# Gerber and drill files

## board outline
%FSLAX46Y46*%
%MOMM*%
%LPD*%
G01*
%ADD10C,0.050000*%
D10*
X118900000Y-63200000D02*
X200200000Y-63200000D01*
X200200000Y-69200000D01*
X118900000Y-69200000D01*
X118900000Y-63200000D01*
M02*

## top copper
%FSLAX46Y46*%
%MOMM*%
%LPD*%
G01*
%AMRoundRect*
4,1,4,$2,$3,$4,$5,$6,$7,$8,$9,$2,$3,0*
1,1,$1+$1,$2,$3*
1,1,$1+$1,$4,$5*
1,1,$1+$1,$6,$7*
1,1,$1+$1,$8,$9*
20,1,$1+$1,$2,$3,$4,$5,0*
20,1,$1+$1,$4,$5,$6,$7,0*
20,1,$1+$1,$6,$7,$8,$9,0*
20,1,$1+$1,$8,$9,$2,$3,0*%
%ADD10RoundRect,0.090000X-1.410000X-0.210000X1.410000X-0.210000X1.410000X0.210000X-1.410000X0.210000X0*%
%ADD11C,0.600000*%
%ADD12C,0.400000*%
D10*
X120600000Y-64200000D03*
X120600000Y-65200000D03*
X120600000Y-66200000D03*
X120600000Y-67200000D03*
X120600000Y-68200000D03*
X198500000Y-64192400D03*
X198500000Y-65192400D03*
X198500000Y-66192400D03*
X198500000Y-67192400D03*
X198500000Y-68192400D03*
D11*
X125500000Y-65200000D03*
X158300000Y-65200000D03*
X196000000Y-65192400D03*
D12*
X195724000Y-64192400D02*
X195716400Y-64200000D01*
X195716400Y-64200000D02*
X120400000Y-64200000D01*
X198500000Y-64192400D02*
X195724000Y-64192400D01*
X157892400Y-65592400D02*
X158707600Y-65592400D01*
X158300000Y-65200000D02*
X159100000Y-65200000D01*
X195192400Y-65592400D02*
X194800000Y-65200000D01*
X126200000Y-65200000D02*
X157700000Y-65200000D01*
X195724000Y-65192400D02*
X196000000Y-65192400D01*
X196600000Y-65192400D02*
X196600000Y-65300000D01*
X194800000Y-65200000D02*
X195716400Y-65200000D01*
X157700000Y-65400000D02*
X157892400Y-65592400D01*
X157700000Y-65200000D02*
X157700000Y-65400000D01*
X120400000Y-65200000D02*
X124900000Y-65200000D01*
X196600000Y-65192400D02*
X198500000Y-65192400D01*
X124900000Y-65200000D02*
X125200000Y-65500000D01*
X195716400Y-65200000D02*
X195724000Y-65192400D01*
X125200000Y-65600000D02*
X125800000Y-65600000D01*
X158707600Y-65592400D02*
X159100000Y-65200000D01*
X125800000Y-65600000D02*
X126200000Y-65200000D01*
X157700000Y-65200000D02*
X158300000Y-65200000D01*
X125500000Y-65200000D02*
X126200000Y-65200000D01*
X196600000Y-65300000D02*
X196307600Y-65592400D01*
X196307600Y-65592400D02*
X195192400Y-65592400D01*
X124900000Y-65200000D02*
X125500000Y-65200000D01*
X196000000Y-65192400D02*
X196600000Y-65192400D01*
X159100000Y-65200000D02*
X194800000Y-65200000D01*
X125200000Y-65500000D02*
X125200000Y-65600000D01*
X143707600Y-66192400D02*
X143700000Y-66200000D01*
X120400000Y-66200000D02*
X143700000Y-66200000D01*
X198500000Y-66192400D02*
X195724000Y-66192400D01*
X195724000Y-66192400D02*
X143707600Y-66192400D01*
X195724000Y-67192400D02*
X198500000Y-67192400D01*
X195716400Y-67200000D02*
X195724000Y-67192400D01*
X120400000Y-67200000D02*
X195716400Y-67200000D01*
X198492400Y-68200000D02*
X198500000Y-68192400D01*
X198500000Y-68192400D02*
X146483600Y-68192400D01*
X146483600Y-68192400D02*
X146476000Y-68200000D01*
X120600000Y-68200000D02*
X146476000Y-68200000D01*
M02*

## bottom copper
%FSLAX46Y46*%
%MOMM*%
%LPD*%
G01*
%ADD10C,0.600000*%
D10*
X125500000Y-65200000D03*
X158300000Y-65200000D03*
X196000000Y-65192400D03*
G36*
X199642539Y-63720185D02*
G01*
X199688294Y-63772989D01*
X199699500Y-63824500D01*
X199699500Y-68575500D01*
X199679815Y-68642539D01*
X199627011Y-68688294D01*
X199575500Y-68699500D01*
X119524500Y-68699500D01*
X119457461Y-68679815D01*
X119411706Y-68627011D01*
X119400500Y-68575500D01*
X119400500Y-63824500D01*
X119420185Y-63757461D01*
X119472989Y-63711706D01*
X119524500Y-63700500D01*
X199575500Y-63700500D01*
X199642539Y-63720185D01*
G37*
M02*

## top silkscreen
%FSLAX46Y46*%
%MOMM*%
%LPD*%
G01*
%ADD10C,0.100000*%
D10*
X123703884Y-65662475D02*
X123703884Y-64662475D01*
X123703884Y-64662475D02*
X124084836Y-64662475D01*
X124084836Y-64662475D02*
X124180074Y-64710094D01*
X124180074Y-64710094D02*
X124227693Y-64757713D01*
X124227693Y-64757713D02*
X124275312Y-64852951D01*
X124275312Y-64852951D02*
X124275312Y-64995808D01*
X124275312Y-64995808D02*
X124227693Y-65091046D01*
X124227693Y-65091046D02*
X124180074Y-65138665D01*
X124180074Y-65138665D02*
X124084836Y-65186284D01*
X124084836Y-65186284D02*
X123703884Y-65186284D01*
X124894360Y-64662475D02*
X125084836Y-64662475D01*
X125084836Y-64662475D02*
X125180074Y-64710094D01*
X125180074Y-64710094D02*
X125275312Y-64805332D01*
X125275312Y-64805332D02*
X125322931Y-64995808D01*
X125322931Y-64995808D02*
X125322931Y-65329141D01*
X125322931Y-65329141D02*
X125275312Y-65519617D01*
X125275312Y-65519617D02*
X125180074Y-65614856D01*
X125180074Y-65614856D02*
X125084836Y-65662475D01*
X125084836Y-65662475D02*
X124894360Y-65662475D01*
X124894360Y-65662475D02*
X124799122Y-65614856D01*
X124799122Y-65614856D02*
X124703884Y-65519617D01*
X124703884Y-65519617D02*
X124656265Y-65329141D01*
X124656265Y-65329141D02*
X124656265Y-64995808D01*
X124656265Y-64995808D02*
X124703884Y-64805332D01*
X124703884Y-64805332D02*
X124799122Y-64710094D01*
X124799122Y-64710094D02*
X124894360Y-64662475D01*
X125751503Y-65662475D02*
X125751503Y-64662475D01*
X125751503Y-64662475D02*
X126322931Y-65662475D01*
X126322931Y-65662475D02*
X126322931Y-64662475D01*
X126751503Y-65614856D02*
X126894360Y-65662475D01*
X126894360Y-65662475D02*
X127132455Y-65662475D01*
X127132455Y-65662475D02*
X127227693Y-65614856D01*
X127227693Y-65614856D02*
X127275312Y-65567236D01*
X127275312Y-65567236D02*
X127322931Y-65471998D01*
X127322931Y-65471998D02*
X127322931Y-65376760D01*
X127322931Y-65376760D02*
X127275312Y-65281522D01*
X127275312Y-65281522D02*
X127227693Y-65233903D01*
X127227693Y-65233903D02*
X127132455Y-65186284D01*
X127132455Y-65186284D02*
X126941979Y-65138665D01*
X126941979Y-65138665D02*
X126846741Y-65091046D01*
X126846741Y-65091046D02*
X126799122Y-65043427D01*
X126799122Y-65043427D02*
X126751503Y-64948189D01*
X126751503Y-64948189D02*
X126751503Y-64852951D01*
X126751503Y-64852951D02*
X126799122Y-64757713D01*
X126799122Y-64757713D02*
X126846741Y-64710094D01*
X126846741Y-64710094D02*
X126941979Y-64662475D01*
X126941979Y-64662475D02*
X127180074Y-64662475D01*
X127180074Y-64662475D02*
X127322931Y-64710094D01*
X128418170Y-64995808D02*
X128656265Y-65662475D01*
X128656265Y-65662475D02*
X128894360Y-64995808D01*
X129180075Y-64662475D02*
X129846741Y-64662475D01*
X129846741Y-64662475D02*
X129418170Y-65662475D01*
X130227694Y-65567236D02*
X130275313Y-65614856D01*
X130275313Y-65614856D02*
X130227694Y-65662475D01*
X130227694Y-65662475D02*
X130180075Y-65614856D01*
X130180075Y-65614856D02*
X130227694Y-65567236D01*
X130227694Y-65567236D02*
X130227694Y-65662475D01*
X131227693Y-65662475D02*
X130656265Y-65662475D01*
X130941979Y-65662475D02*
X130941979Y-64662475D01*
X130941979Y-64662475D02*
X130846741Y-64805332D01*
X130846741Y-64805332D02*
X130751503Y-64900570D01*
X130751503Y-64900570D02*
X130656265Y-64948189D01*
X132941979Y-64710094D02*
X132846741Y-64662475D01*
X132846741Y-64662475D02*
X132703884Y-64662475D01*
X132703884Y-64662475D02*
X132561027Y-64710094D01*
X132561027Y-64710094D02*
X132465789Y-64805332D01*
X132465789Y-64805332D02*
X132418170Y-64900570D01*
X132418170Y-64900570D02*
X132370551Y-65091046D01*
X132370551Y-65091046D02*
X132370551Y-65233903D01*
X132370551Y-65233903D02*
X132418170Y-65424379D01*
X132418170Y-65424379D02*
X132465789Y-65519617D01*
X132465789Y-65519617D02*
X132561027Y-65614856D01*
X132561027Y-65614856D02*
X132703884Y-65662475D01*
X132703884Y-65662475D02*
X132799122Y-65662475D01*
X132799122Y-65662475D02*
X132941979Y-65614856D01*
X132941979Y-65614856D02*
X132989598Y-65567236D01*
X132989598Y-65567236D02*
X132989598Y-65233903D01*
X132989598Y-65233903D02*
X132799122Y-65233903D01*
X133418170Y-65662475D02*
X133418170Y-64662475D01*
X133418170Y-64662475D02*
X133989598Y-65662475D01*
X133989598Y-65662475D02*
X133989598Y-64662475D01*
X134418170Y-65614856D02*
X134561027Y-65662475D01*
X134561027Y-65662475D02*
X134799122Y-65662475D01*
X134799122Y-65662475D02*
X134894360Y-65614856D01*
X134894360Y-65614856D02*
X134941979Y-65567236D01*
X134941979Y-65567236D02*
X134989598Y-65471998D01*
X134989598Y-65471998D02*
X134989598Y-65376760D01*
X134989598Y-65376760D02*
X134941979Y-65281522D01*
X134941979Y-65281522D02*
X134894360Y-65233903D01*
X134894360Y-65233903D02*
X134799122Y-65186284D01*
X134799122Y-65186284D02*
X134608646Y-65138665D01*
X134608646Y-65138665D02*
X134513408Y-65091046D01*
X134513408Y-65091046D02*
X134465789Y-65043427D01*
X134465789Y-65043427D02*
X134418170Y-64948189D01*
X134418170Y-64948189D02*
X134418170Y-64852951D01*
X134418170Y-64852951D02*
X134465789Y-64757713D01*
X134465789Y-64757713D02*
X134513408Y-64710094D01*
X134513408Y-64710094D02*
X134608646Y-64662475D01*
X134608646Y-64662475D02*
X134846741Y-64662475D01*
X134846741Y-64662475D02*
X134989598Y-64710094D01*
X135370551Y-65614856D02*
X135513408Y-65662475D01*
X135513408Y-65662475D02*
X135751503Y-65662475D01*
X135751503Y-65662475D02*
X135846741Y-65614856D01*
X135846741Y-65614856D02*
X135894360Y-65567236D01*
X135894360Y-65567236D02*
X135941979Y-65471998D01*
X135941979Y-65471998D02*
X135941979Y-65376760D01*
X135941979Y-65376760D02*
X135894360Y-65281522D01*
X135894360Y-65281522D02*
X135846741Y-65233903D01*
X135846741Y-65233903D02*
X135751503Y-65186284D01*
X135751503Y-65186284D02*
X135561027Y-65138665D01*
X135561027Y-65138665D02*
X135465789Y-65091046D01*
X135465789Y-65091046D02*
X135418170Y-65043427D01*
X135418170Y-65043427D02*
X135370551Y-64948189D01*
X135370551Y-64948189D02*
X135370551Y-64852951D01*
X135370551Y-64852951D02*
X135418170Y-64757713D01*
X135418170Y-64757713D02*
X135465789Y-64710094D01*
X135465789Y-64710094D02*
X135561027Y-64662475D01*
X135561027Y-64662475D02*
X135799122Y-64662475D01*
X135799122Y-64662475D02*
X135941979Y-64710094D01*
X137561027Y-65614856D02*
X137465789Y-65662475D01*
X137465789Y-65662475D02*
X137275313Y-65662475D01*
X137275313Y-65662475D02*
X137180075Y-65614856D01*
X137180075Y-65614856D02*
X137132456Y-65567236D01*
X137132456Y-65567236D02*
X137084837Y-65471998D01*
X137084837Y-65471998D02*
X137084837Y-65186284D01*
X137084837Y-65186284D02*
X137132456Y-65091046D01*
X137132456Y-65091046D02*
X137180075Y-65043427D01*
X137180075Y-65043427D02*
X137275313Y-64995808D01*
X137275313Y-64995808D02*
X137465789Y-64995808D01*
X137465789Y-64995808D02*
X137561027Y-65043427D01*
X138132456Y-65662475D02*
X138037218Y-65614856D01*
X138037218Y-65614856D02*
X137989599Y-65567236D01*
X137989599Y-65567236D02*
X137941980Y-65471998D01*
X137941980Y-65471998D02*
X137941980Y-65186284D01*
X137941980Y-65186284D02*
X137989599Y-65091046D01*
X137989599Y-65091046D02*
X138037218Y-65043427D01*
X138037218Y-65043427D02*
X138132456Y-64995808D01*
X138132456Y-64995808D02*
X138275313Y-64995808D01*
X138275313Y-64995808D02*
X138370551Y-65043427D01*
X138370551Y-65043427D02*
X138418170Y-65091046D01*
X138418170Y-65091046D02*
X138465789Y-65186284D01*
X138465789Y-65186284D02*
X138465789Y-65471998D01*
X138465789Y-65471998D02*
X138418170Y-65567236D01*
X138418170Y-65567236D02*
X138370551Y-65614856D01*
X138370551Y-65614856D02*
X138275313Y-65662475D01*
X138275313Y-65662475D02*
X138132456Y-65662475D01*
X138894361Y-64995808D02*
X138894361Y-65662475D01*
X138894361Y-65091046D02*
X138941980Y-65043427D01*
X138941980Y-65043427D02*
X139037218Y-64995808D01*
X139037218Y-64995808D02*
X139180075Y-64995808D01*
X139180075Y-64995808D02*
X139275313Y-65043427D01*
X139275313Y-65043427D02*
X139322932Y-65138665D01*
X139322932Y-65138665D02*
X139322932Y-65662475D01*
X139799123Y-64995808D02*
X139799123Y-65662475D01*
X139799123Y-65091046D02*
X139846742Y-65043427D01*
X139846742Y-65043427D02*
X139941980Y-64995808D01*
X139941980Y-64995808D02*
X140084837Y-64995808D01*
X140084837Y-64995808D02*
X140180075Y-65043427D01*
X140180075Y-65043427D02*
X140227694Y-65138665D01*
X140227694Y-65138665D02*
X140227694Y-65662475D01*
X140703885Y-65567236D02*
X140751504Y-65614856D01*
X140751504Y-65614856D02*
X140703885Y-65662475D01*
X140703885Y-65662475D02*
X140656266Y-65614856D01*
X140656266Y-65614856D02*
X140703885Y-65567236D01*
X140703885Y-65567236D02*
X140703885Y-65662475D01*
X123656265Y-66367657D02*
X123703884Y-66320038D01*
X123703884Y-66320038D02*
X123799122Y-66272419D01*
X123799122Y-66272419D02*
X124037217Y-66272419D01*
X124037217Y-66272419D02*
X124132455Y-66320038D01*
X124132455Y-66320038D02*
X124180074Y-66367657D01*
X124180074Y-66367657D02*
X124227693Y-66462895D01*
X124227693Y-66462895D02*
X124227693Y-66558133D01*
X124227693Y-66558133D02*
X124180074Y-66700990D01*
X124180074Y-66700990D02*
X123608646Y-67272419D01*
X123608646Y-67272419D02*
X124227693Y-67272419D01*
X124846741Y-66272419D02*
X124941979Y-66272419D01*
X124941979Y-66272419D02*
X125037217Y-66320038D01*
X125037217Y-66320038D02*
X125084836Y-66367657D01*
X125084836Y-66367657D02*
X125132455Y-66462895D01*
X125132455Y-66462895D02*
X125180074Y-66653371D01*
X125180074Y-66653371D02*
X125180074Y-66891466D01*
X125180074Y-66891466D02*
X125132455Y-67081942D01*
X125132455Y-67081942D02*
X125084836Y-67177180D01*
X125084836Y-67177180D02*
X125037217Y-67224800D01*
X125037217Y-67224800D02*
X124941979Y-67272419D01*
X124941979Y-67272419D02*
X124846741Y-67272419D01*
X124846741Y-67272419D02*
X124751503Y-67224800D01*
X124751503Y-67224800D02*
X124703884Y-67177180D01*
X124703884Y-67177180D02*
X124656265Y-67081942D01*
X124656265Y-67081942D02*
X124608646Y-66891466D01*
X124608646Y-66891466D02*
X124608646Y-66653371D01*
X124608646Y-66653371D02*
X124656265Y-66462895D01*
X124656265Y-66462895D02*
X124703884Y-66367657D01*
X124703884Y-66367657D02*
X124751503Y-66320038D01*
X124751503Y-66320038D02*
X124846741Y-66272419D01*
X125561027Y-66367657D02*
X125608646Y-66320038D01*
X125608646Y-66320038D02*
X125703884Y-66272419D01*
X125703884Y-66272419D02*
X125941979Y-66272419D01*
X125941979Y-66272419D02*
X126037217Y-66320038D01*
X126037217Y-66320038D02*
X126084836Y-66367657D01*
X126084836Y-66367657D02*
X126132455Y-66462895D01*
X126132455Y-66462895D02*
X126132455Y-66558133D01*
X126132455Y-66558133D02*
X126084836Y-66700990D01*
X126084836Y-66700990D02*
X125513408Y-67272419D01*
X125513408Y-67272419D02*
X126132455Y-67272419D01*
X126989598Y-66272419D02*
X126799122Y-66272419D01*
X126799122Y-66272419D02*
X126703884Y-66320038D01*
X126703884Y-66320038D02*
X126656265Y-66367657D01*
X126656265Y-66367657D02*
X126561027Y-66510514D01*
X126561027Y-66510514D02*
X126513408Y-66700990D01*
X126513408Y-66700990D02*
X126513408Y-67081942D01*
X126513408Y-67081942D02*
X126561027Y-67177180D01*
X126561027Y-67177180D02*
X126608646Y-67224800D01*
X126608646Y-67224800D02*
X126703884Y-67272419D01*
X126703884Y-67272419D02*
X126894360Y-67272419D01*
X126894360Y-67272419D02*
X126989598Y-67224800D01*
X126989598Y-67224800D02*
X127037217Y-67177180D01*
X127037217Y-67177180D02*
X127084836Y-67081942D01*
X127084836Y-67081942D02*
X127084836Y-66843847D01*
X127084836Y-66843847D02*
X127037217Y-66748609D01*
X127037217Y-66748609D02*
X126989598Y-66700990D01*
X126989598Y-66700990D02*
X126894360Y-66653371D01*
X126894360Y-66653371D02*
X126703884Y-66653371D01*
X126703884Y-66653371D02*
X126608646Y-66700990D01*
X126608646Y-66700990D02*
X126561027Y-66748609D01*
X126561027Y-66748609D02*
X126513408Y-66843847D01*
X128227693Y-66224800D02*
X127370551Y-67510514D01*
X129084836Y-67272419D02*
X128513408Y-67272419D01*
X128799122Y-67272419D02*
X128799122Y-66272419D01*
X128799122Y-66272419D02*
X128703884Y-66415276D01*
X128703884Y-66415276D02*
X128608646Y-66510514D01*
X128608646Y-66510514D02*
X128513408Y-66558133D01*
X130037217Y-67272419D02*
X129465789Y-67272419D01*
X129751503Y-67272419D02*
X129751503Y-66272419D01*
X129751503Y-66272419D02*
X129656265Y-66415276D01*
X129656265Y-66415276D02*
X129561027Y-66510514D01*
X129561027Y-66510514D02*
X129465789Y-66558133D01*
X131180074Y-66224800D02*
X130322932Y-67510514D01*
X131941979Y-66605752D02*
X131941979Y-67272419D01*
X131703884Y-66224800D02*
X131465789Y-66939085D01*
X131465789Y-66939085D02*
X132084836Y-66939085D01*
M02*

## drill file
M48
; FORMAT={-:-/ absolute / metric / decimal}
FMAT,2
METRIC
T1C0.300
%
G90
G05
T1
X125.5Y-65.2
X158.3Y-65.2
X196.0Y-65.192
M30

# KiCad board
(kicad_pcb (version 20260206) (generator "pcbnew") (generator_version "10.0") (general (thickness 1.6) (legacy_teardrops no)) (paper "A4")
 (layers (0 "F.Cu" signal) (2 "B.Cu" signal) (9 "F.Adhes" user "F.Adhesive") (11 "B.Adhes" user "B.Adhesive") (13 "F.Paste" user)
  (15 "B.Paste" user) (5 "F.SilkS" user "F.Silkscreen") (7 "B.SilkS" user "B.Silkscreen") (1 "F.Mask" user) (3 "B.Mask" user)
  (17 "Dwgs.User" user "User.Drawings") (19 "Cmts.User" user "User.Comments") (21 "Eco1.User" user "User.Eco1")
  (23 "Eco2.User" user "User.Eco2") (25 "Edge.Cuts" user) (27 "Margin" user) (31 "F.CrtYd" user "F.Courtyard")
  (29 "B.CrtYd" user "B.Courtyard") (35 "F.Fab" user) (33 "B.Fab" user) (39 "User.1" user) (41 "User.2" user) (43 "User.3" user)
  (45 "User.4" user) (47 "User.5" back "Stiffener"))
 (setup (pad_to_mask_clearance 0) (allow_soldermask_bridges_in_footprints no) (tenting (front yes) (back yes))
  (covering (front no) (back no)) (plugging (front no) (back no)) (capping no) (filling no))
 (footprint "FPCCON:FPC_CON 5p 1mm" (layer "F.Cu") (at 120.6 66.2)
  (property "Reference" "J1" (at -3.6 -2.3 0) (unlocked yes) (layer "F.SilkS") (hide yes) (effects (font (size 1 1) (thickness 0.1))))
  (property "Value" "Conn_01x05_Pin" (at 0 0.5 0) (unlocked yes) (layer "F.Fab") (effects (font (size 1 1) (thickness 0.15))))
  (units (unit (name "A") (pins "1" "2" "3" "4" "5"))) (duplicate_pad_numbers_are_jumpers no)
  (pad "1" smd roundrect (at 0 -2) (size 3 0.6) (layers "F.Cu" "F.Mask" "F.Paste") (roundrect_rratio 0.15) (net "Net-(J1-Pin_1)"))
  (pad "2" smd roundrect (at 0 -1) (size 3 0.6) (layers "F.Cu" "F.Mask" "F.Paste") (roundrect_rratio 0.15) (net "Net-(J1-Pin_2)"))
  (pad "3" smd roundrect (at 0 0) (size 3 0.6) (layers "F.Cu" "F.Mask" "F.Paste") (roundrect_rratio 0.15) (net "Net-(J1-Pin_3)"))
  (pad "4" smd roundrect (at 0 1) (size 3 0.6) (layers "F.Cu" "F.Mask" "F.Paste") (roundrect_rratio 0.15) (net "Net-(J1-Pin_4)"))
  (pad "5" smd roundrect (at 0 2) (size 3 0.6) (layers "F.Cu" "F.Mask" "F.Paste") (roundrect_rratio 0.15) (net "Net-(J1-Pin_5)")))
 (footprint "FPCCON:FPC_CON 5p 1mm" (layer "F.Cu") (at 198.5 66.1924)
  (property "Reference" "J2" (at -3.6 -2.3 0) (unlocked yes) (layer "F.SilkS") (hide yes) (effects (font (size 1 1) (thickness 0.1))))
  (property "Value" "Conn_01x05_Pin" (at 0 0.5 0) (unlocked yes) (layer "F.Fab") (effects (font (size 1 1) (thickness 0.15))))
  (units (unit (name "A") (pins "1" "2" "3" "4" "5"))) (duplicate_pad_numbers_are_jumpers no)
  (pad "1" smd roundrect (at 0 -2) (size 3 0.6) (layers "F.Cu" "F.Mask" "F.Paste") (roundrect_rratio 0.15) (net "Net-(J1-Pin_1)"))
  (pad "2" smd roundrect (at 0 -1) (size 3 0.6) (layers "F.Cu" "F.Mask" "F.Paste") (roundrect_rratio 0.15) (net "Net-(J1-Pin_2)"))
  (pad "3" smd roundrect (at 0 0) (size 3 0.6) (layers "F.Cu" "F.Mask" "F.Paste") (roundrect_rratio 0.15) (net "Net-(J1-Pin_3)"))
  (pad "4" smd roundrect (at 0 1) (size 3 0.6) (layers "F.Cu" "F.Mask" "F.Paste") (roundrect_rratio 0.15) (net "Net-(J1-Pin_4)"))
  (pad "5" smd roundrect (at 0 2) (size 3 0.6) (layers "F.Cu" "F.Mask" "F.Paste") (roundrect_rratio 0.15) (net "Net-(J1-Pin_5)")))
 (gr_rect (start 118.9 63.2) (end 200.2 69.2) (stroke (width 0.05) (type default)) (fill no) (layer "Edge.Cuts"))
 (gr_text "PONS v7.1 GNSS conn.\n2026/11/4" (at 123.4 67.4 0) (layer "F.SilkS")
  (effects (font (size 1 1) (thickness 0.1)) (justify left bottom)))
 (segment (start 195.724 64.1924) (end 195.7164 64.2) (width 0.4) (layer "F.Cu") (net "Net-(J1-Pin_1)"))
 (segment (start 195.7164 64.2) (end 120.4 64.2) (width 0.4) (layer "F.Cu") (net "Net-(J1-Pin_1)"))
 (segment (start 198.5 64.1924) (end 195.724 64.1924) (width 0.4) (layer "F.Cu") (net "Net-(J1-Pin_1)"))
 (segment (start 157.8924 65.5924) (end 158.7076 65.5924) (width 0.4) (layer "F.Cu") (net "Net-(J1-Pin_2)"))
 (segment (start 158.3 65.2) (end 159.1 65.2) (width 0.4) (layer "F.Cu") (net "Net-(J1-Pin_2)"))
 (segment (start 195.1924 65.5924) (end 194.8 65.2) (width 0.4) (layer "F.Cu") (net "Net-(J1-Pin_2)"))
 (segment (start 126.2 65.2) (end 157.7 65.2) (width 0.4) (layer "F.Cu") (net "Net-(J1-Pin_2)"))
 (segment (start 195.724 65.1924) (end 196 65.1924) (width 0.4) (layer "F.Cu") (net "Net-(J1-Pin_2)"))
 (segment (start 196.6 65.1924) (end 196.6 65.3) (width 0.4) (layer "F.Cu") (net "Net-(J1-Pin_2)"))
 (segment (start 194.8 65.2) (end 195.7164 65.2) (width 0.4) (layer "F.Cu") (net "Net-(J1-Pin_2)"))
 (segment (start 157.7 65.4) (end 157.8924 65.5924) (width 0.4) (layer "F.Cu") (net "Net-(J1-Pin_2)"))
 (segment (start 157.7 65.2) (end 157.7 65.4) (width 0.4) (layer "F.Cu") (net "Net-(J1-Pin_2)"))
 (segment (start 120.4 65.2) (end 124.9 65.2) (width 0.4) (layer "F.Cu") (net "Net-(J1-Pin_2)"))
 (segment (start 196.6 65.1924) (end 198.5 65.1924) (width 0.4) (layer "F.Cu") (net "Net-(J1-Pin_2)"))
 (segment (start 124.9 65.2) (end 125.2 65.5) (width 0.4) (layer "F.Cu") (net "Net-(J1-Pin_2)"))
 (segment (start 195.7164 65.2) (end 195.724 65.1924) (width 0.4) (layer "F.Cu") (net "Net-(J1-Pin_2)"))
 (segment (start 125.2 65.6) (end 125.8 65.6) (width 0.4) (layer "F.Cu") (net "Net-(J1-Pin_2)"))
 (segment (start 158.7076 65.5924) (end 159.1 65.2) (width 0.4) (layer "F.Cu") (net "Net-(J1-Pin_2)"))
 (segment (start 125.8 65.6) (end 126.2 65.2) (width 0.4) (layer "F.Cu") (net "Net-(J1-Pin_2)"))
 (segment (start 157.7 65.2) (end 158.3 65.2) (width 0.4) (layer "F.Cu") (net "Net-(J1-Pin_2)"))
 (segment (start 125.5 65.2) (end 126.2 65.2) (width 0.4) (layer "F.Cu") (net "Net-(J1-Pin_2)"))
 (segment (start 196.6 65.3) (end 196.3076 65.5924) (width 0.4) (layer "F.Cu") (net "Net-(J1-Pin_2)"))
 (segment (start 196.3076 65.5924) (end 195.1924 65.5924) (width 0.4) (layer "F.Cu") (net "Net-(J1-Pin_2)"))
 (segment (start 124.9 65.2) (end 125.5 65.2) (width 0.4) (layer "F.Cu") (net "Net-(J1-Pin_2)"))
 (segment (start 196 65.1924) (end 196.6 65.1924) (width 0.4) (layer "F.Cu") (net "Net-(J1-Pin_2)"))
 (segment (start 159.1 65.2) (end 194.8 65.2) (width 0.4) (layer "F.Cu") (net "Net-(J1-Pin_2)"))
 (segment (start 125.2 65.5) (end 125.2 65.6) (width 0.4) (layer "F.Cu") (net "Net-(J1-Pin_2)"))
 (via (at 125.5 65.2) (size 0.6) (drill 0.3) (layers "F.Cu" "B.Cu") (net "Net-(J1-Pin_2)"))
 (via (at 158.3 65.2) (size 0.6) (drill 0.3) (layers "F.Cu" "B.Cu") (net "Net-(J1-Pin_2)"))
 (via (at 196 65.1924) (size 0.6) (drill 0.3) (layers "F.Cu" "B.Cu") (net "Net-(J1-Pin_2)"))
 (segment (start 143.7076 66.1924) (end 143.7 66.2) (width 0.4) (layer "F.Cu") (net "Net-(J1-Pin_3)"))
 (segment (start 120.4 66.2) (end 143.7 66.2) (width 0.4) (layer "F.Cu") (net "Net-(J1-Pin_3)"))
 (segment (start 198.5 66.1924) (end 195.724 66.1924) (width 0.4) (layer "F.Cu") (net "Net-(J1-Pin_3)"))
 (segment (start 195.724 66.1924) (end 143.7076 66.1924) (width 0.4) (layer "F.Cu") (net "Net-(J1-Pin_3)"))
 (segment (start 195.724 67.1924) (end 198.5 67.1924) (width 0.4) (layer "F.Cu") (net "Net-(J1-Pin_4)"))
 (segment (start 195.7164 67.2) (end 195.724 67.1924) (width 0.4) (layer "F.Cu") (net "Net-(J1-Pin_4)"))
 (segment (start 120.4 67.2) (end 195.7164 67.2) (width 0.4) (layer "F.Cu") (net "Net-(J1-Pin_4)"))
 (segment (start 198.4924 68.2) (end 198.5 68.1924) (width 0.4) (layer "F.Cu") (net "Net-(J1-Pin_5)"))
 (segment (start 198.5 68.1924) (end 146.4836 68.1924) (width 0.4) (layer "F.Cu") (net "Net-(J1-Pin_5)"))
 (segment (start 146.4836 68.1924) (end 146.476 68.2) (width 0.4) (layer "F.Cu") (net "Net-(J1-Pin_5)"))
 (segment (start 120.6 68.2) (end 146.476 68.2) (width 0.4) (layer "F.Cu") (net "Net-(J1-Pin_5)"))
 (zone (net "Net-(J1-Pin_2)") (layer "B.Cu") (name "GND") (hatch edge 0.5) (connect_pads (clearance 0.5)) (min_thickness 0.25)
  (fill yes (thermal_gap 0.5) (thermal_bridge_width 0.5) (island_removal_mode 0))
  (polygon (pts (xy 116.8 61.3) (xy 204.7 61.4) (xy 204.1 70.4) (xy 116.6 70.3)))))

